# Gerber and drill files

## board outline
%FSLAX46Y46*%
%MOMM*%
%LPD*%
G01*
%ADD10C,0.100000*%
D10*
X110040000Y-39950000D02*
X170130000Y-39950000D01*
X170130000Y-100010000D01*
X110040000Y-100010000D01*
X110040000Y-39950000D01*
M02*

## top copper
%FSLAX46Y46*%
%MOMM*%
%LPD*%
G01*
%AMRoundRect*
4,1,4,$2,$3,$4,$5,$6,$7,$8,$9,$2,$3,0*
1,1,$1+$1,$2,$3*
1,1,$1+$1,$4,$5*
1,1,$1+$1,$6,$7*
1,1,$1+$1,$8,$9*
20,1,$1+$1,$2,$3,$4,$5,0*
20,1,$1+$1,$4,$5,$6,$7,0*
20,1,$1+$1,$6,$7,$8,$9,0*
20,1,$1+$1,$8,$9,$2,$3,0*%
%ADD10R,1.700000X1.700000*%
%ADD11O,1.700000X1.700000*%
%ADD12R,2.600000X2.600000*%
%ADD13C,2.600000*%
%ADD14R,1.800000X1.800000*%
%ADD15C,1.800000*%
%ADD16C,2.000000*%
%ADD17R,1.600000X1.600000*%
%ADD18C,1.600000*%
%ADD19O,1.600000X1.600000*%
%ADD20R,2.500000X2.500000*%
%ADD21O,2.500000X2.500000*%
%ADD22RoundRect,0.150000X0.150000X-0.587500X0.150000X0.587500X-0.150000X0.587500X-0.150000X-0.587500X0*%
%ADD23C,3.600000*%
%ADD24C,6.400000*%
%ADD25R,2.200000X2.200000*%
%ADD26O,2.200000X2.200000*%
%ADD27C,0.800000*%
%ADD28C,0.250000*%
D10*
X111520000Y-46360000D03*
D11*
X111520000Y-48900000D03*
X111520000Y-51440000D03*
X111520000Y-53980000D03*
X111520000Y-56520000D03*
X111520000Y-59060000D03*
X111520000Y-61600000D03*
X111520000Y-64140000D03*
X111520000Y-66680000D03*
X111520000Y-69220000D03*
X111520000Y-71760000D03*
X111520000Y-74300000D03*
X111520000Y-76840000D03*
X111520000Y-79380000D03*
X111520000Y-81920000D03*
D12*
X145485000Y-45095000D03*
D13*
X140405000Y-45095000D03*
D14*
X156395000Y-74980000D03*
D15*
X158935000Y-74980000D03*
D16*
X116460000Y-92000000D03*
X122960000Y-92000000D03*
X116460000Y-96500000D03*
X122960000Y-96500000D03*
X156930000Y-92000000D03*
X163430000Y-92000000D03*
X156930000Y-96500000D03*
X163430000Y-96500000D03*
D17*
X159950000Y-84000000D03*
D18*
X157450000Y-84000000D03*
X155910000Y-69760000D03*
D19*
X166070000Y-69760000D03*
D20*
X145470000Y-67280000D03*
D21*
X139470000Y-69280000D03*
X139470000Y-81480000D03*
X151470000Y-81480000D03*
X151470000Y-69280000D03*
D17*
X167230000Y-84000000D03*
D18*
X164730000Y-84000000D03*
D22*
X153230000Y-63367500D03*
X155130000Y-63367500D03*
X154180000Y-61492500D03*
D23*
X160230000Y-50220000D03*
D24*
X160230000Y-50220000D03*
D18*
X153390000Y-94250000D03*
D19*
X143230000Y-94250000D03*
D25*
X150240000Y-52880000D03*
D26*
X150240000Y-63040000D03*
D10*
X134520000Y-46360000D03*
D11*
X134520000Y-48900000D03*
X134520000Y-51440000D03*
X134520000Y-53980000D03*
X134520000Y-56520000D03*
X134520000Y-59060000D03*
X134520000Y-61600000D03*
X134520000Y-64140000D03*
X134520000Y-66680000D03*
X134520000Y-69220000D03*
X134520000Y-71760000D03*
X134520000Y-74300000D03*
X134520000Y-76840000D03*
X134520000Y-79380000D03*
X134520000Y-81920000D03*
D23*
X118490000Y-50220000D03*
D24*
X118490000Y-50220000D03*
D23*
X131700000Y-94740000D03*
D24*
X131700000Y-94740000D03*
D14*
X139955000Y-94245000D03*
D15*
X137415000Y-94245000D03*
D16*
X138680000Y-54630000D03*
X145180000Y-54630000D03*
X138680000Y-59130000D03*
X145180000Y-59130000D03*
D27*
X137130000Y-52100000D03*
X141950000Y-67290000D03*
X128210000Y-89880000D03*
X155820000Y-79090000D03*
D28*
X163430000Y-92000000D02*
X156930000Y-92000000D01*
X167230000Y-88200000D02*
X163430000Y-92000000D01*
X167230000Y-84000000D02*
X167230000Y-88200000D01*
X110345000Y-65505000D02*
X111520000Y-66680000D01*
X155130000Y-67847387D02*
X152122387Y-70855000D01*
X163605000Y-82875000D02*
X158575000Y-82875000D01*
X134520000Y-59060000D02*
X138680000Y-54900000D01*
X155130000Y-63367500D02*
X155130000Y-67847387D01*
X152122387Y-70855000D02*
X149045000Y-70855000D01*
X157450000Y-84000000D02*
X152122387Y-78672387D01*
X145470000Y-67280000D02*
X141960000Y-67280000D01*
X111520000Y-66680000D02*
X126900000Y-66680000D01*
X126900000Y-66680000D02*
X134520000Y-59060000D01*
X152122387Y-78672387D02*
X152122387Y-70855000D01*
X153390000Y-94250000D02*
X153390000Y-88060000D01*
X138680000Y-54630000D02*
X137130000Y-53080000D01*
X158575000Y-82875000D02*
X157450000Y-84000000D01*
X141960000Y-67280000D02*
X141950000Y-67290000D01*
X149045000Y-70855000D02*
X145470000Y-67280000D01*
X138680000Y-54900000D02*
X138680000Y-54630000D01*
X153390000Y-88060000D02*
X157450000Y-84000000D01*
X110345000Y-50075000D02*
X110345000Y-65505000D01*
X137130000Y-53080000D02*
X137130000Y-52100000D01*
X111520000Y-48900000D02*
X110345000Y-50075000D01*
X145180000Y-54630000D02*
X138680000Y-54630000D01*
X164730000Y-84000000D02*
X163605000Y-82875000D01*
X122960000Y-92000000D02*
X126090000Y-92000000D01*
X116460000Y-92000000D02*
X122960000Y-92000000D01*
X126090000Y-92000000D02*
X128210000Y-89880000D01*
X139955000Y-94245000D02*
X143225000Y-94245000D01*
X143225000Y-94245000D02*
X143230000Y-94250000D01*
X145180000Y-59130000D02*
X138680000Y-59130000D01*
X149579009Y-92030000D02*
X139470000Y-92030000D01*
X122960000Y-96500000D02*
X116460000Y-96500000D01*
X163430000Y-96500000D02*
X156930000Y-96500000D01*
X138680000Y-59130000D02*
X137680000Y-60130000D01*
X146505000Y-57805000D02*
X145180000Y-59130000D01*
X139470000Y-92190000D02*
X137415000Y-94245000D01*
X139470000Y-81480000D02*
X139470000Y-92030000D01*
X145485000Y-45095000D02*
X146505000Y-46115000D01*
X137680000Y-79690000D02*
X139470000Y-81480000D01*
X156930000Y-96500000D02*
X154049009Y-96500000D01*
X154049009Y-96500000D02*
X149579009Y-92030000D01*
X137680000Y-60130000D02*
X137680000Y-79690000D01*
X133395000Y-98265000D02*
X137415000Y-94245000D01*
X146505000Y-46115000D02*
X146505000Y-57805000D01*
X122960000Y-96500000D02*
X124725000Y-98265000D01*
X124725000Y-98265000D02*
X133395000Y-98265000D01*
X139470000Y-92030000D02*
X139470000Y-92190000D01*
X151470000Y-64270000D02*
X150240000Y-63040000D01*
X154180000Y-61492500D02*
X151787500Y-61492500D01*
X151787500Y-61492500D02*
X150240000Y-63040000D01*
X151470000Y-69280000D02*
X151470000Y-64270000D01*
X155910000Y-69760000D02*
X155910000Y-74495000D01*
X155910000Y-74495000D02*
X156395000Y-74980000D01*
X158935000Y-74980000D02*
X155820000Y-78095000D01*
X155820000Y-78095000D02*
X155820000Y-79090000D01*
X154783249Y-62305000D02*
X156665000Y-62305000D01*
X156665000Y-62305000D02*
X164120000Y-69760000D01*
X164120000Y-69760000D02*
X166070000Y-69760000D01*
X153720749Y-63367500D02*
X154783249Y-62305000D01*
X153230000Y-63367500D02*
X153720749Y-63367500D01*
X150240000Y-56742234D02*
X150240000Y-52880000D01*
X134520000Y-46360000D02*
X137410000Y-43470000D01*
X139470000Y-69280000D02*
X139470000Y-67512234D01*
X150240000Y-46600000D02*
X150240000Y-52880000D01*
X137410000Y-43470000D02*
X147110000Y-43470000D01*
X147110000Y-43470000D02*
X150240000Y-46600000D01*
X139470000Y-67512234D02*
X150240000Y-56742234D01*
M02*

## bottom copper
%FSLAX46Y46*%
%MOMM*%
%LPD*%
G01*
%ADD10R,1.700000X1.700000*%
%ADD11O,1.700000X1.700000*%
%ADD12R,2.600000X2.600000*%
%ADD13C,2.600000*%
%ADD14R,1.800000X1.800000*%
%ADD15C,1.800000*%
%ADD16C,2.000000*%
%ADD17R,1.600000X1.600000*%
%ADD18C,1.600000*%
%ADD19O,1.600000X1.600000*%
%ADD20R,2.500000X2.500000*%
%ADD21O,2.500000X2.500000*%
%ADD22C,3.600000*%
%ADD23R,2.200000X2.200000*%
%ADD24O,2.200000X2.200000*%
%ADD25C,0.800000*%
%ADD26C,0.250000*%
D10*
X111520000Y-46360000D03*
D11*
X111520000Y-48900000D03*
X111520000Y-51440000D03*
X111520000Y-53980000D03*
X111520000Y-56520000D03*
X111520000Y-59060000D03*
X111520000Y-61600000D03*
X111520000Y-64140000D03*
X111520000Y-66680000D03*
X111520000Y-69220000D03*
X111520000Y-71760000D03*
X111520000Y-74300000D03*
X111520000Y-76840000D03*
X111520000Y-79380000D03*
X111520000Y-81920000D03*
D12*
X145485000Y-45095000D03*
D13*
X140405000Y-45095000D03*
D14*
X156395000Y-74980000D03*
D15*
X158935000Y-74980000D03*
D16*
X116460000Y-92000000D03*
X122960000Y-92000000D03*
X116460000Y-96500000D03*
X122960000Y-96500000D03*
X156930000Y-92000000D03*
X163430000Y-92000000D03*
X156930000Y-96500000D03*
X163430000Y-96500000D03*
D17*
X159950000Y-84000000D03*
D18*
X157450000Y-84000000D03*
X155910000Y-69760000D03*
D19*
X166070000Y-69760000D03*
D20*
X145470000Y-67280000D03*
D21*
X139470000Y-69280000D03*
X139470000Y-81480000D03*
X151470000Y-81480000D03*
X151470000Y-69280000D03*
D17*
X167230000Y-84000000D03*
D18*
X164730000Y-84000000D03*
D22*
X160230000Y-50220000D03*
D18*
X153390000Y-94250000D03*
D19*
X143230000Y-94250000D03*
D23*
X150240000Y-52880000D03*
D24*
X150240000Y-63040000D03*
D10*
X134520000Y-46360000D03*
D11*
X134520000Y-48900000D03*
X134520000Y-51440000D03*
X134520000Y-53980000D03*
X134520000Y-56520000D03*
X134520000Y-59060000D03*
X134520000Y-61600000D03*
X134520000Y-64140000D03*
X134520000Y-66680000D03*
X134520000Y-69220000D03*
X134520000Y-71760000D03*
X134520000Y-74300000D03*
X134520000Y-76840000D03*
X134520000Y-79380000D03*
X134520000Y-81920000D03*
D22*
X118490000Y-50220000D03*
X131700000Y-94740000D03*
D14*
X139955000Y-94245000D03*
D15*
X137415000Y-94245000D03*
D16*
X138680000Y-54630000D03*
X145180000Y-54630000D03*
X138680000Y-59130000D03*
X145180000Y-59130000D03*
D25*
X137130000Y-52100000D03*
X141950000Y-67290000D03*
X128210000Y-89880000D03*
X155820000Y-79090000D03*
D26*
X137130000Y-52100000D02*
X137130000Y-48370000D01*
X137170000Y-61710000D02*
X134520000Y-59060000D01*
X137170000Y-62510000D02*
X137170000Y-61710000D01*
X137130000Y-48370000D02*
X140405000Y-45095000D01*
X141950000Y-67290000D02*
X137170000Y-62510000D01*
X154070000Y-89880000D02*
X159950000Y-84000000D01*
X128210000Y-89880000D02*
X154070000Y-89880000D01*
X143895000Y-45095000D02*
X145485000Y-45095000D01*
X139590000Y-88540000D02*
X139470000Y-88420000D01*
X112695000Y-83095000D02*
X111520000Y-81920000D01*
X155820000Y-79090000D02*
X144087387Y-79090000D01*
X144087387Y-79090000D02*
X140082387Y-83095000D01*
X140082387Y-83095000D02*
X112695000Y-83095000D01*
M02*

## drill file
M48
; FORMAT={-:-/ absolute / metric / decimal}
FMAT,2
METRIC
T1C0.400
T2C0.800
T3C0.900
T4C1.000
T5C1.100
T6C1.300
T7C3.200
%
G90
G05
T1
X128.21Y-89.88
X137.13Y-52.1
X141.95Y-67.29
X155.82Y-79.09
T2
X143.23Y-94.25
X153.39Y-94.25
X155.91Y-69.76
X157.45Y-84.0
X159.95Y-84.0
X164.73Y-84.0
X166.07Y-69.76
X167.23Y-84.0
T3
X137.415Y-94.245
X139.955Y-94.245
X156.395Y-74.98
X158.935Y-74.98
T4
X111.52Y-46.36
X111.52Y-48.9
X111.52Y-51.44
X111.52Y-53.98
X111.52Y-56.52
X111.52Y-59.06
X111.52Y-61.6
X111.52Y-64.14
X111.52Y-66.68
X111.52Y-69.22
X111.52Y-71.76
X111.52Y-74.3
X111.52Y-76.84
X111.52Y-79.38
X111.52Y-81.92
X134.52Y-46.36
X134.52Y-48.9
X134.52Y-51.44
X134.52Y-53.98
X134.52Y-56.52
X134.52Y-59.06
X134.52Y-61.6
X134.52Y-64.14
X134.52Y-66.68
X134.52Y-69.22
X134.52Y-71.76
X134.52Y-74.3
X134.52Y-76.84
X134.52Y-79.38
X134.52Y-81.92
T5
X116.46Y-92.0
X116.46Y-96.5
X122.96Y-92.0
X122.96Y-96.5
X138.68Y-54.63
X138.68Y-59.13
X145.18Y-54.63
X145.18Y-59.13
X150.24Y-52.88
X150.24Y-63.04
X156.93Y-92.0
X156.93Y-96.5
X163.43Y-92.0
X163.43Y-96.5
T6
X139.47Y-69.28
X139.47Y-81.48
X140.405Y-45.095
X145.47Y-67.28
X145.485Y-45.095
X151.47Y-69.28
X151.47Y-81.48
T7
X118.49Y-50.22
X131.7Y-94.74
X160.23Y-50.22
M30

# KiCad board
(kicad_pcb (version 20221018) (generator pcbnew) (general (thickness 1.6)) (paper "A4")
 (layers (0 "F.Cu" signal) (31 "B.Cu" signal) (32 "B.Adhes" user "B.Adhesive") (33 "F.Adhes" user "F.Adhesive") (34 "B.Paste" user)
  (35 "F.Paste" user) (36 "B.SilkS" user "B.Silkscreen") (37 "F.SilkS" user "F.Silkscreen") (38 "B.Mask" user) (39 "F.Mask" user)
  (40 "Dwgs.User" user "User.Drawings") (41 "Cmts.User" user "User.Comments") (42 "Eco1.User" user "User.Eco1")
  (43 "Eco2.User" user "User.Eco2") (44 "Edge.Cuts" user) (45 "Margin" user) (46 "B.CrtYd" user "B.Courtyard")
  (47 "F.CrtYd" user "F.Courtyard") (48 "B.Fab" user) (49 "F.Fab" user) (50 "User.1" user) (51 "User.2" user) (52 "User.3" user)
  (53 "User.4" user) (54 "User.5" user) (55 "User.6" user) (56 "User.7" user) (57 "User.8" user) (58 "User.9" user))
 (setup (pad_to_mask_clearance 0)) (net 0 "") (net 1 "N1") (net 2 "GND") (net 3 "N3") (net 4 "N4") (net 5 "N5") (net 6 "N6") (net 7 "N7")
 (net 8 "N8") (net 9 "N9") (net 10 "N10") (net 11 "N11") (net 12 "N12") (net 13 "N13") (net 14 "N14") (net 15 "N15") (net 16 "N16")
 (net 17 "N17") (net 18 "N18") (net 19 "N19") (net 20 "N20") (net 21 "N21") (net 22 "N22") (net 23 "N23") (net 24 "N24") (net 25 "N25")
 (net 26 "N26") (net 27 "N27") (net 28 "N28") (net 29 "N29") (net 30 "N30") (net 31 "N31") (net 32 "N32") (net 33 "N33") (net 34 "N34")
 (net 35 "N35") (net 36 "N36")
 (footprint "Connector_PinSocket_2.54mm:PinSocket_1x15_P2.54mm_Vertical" (layer "F.Cu") (at 111.52 46.36)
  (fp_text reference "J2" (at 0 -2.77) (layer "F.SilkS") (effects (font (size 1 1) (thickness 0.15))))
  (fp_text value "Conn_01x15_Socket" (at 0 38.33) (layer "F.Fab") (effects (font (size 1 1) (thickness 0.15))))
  (pad "1" thru_hole rect (at 0 0) (size 1.7 1.7) (drill 1) (layers "*.Cu" "*.Mask") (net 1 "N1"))
  (pad "2" thru_hole oval (at 0 2.54) (size 1.7 1.7) (drill 1) (layers "*.Cu" "*.Mask") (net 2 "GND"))
  (pad "3" thru_hole oval (at 0 5.08) (size 1.7 1.7) (drill 1) (layers "*.Cu" "*.Mask") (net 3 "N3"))
  (pad "4" thru_hole oval (at 0 7.62) (size 1.7 1.7) (drill 1) (layers "*.Cu" "*.Mask") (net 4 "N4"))
  (pad "5" thru_hole oval (at 0 10.16) (size 1.7 1.7) (drill 1) (layers "*.Cu" "*.Mask") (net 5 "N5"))
  (pad "6" thru_hole oval (at 0 12.7) (size 1.7 1.7) (drill 1) (layers "*.Cu" "*.Mask") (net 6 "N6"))
  (pad "7" thru_hole oval (at 0 15.24) (size 1.7 1.7) (drill 1) (layers "*.Cu" "*.Mask") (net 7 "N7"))
  (pad "8" thru_hole oval (at 0 17.78) (size 1.7 1.7) (drill 1) (layers "*.Cu" "*.Mask") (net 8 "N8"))
  (pad "9" thru_hole oval (at 0 20.32) (size 1.7 1.7) (drill 1) (layers "*.Cu" "*.Mask") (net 2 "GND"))
  (pad "10" thru_hole oval (at 0 22.86) (size 1.7 1.7) (drill 1) (layers "*.Cu" "*.Mask") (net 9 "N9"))
  (pad "11" thru_hole oval (at 0 25.4) (size 1.7 1.7) (drill 1) (layers "*.Cu" "*.Mask") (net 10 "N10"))
  (pad "12" thru_hole oval (at 0 27.94) (size 1.7 1.7) (drill 1) (layers "*.Cu" "*.Mask") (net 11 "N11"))
  (pad "13" thru_hole oval (at 0 30.48) (size 1.7 1.7) (drill 1) (layers "*.Cu" "*.Mask") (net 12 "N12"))
  (pad "14" thru_hole oval (at 0 33.02) (size 1.7 1.7) (drill 1) (layers "*.Cu" "*.Mask") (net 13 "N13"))
  (pad "15" thru_hole oval (at 0 35.56) (size 1.7 1.7) (drill 1) (layers "*.Cu" "*.Mask") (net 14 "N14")))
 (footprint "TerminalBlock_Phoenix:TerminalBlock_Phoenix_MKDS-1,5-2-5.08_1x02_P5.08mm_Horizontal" (layer "F.Cu") (at 145.485 45.095 180)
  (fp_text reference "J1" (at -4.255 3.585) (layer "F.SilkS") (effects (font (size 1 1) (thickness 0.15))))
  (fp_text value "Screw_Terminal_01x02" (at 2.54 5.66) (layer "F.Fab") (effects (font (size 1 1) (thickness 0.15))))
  (pad "1" thru_hole rect (at 0 0 180) (size 2.6 2.6) (drill 1.3) (layers "*.Cu" "*.Mask") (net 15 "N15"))
  (pad "2" thru_hole circle (at 5.08 0 180) (size 2.6 2.6) (drill 1.3) (layers "*.Cu" "*.Mask") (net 2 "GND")))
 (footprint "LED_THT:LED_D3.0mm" (layer "F.Cu") (at 156.395 74.98)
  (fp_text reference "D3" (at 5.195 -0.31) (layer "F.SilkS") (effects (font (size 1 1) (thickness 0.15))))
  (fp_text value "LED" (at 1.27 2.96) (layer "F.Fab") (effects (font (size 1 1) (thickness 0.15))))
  (pad "1" thru_hole rect (at 0 0) (size 1.8 1.8) (drill 0.9) (layers "*.Cu" "*.Mask") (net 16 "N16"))
  (pad "2" thru_hole circle (at 2.54 0) (size 1.8 1.8) (drill 0.9) (layers "*.Cu" "*.Mask") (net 14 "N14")))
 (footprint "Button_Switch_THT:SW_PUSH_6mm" (layer "F.Cu") (at 116.46 92)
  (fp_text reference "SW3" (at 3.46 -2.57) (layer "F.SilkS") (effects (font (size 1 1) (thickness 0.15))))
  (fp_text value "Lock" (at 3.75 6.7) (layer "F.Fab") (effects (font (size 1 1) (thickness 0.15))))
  (pad "1" thru_hole circle (at 0 0 90) (size 2 2) (drill 1.1) (layers "*.Cu" "*.Mask") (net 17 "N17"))
  (pad "1" thru_hole circle (at 6.5 0 90) (size 2 2) (drill 1.1) (layers "*.Cu" "*.Mask") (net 17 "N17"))
  (pad "2" thru_hole circle (at 0 4.5 90) (size 2 2) (drill 1.1) (layers "*.Cu" "*.Mask") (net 15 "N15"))
  (pad "2" thru_hole circle (at 6.5 4.5 90) (size 2 2) (drill 1.1) (layers "*.Cu" "*.Mask") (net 15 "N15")))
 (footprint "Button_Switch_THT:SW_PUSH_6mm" (layer "F.Cu") (at 156.93 92)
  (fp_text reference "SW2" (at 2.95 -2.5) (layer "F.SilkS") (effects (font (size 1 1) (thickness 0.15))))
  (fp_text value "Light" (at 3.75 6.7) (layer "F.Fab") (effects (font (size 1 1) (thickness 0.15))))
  (pad "1" thru_hole circle (at 0 0 90) (size 2 2) (drill 1.1) (layers "*.Cu" "*.Mask") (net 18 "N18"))
  (pad "1" thru_hole circle (at 6.5 0 90) (size 2 2) (drill 1.1) (layers "*.Cu" "*.Mask") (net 18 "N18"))
  (pad "2" thru_hole circle (at 0 4.5 90) (size 2 2) (drill 1.1) (layers "*.Cu" "*.Mask") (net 15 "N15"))
  (pad "2" thru_hole circle (at 6.5 4.5 90) (size 2 2) (drill 1.1) (layers "*.Cu" "*.Mask") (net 15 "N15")))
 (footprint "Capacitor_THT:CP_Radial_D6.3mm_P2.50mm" (layer "F.Cu") (at 159.95 84 180)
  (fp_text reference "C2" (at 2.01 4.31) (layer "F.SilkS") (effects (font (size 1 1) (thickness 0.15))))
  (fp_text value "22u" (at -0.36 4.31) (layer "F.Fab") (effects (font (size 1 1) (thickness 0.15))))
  (pad "1" thru_hole rect (at 0 0 180) (size 1.6 1.6) (drill 0.8) (layers "*.Cu" "*.Mask") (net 17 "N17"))
  (pad "2" thru_hole circle (at 2.5 0 180) (size 1.6 1.6) (drill 0.8) (layers "*.Cu" "*.Mask") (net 2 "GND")))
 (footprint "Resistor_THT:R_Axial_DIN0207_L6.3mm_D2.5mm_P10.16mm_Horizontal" (layer "F.Cu") (at 155.91 69.76)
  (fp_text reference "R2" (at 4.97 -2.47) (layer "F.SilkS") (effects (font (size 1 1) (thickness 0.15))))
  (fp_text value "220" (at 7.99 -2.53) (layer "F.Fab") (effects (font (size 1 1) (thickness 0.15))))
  (pad "1" thru_hole circle (at 0 0) (size 1.6 1.6) (drill 0.8) (layers "*.Cu" "*.Mask") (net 16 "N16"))
  (pad "2" thru_hole oval (at 10.16 0) (size 1.6 1.6) (drill 0.8) (layers "*.Cu" "*.Mask") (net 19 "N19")))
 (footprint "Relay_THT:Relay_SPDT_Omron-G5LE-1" (layer "F.Cu") (at 145.47 67.28)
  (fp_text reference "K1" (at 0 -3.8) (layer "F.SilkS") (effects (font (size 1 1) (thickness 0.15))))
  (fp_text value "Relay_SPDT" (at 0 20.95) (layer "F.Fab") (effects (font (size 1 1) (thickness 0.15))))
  (pad "1" thru_hole rect (at 0 0) (size 2.5 2.5) (drill 1.3) (layers "*.Cu" "*.Mask") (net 2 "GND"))
  (pad "2" thru_hole oval (at -6 2) (size 2.5 2.5) (drill 1.3) (layers "*.Cu" "*.Mask") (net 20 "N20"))
  (pad "3" thru_hole oval (at -6 14.2) (size 2.5 2.5) (drill 1.3) (layers "*.Cu" "*.Mask") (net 15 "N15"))
  (pad "4" thru_hole oval (at 6 14.2) (size 2.5 2.5) (drill 1.3) (layers "*.Cu" "*.Mask") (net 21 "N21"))
  (pad "5" thru_hole oval (at 6 2) (size 2.5 2.5) (drill 1.3) (layers "*.Cu" "*.Mask") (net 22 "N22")))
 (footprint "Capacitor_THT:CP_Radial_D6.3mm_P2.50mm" (layer "F.Cu") (at 167.23 84 180)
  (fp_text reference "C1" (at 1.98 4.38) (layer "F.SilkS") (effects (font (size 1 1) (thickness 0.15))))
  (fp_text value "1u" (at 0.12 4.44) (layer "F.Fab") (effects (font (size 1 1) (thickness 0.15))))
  (pad "1" thru_hole rect (at 0 0 180) (size 1.6 1.6) (drill 0.8) (layers "*.Cu" "*.Mask") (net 18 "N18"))
  (pad "2" thru_hole circle (at 2.5 0 180) (size 1.6 1.6) (drill 0.8) (layers "*.Cu" "*.Mask") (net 2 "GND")))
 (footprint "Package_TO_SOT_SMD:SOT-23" (layer "F.Cu") (at 154.18 62.43 90)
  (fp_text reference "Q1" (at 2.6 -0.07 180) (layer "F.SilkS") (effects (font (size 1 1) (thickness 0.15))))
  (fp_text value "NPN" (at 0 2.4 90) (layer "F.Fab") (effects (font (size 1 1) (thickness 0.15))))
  (pad "1" smd roundrect (at -0.9375 -0.95 90) (size 1.475 0.6) (layers "F.Cu" "F.Paste" "F.Mask") (roundrect_rratio 0.25) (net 19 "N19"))
  (pad "2" smd roundrect (at -0.9375 0.95 90) (size 1.475 0.6) (layers "F.Cu" "F.Paste" "F.Mask") (roundrect_rratio 0.25) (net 2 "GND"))
  (pad "3" smd roundrect (at 0.9375 0 90) (size 1.475 0.6) (layers "F.Cu" "F.Paste" "F.Mask") (roundrect_rratio 0.25) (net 22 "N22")))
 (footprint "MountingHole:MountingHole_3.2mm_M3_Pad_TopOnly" (layer "F.Cu") (at 160.23 50.22)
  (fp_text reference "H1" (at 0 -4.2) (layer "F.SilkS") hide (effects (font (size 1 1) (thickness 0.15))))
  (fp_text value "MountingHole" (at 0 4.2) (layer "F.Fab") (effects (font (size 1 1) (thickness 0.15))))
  (pad "1" thru_hole circle (at 0 0) (size 3.6 3.6) (drill 3.2) (layers "*.Cu" "*.Mask"))
  (pad "1" connect circle (at 0 0) (size 6.4 6.4) (layers "F.Cu" "F.Mask")))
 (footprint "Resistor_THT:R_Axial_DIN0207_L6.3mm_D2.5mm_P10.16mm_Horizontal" (layer "F.Cu") (at 153.39 94.25 180)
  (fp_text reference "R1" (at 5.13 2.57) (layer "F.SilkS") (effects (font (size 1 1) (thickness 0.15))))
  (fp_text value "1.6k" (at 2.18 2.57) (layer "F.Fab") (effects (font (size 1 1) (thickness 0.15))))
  (pad "1" thru_hole circle (at 0 0 180) (size 1.6 1.6) (drill 0.8) (layers "*.Cu" "*.Mask") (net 2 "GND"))
  (pad "2" thru_hole oval (at 10.16 0 180) (size 1.6 1.6) (drill 0.8) (layers "*.Cu" "*.Mask") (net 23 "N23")))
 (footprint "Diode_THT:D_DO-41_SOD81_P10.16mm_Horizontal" (layer "F.Cu") (at 150.24 52.88 -90)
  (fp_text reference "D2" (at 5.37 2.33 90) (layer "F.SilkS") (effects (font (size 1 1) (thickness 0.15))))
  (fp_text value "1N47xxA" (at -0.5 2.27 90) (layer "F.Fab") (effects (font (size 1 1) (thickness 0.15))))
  (pad "1" thru_hole rect (at 0 0 270) (size 2.2 2.2) (drill 1.1) (layers "*.Cu" "*.Mask") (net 20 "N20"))
  (pad "2" thru_hole oval (at 10.16 0 270) (size 2.2 2.2) (drill 1.1) (layers "*.Cu" "*.Mask") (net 22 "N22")))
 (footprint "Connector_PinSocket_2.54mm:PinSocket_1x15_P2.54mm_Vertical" (layer "F.Cu") (at 134.52 46.36)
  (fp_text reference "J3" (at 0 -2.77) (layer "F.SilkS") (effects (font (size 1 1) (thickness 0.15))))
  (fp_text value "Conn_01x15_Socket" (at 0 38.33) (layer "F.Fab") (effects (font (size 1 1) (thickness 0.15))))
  (pad "1" thru_hole rect (at 0 0) (size 1.7 1.7) (drill 1) (layers "*.Cu" "*.Mask") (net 20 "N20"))
  (pad "2" thru_hole oval (at 0 2.54) (size 1.7 1.7) (drill 1) (layers "*.Cu" "*.Mask") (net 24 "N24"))
  (pad "3" thru_hole oval (at 0 5.08) (size 1.7 1.7) (drill 1) (layers "*.Cu" "*.Mask") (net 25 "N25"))
  (pad "4" thru_hole oval (at 0 7.62) (size 1.7 1.7) (drill 1) (layers "*.Cu" "*.Mask") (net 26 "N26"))
  (pad "5" thru_hole oval (at 0 10.16) (size 1.7 1.7) (drill 1) (layers "*.Cu" "*.Mask") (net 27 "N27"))
  (pad "6" thru_hole oval (at 0 12.7) (size 1.7 1.7) (drill 1) (layers "*.Cu" "*.Mask") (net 2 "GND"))
  (pad "7" thru_hole oval (at 0 15.24) (size 1.7 1.7) (drill 1) (layers "*.Cu" "*.Mask") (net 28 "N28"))
  (pad "8" thru_hole oval (at 0 17.78) (size 1.7 1.7) (drill 1) (layers "*.Cu" "*.Mask") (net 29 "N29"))
  (pad "9" thru_hole oval (at 0 20.32) (size 1.7 1.7) (drill 1) (layers "*.Cu" "*.Mask") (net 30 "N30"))
  (pad "10" thru_hole oval (at 0 22.86) (size 1.7 1.7) (drill 1) (layers "*.Cu" "*.Mask") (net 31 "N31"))
  (pad "11" thru_hole oval (at 0 25.4) (size 1.7 1.7) (drill 1) (layers "*.Cu" "*.Mask") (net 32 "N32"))
  (pad "12" thru_hole oval (at 0 27.94) (size 1.7 1.7) (drill 1) (layers "*.Cu" "*.Mask") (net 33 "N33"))
  (pad "13" thru_hole oval (at 0 30.48) (size 1.7 1.7) (drill 1) (layers "*.Cu" "*.Mask") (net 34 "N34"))
  (pad "14" thru_hole oval (at 0 33.02) (size 1.7 1.7) (drill 1) (layers "*.Cu" "*.Mask") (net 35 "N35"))
  (pad "15" thru_hole oval (at 0 35.56) (size 1.7 1.7) (drill 1) (layers "*.Cu" "*.Mask") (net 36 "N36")))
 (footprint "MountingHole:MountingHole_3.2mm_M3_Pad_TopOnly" (layer "F.Cu") (at 118.49 50.22)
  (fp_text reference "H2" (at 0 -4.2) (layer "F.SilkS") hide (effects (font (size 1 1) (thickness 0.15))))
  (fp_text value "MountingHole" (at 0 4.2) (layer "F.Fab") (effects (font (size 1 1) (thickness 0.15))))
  (pad "1" thru_hole circle (at 0 0) (size 3.6 3.6) (drill 3.2) (layers "*.Cu" "*.Mask"))
  (pad "1" connect circle (at 0 0) (size 6.4 6.4) (layers "F.Cu" "F.Mask")))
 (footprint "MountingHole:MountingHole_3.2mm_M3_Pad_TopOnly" (layer "F.Cu") (at 131.7 94.74)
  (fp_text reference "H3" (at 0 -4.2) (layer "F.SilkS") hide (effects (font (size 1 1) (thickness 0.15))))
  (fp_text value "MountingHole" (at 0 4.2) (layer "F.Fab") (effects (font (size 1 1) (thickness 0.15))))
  (pad "1" thru_hole circle (at 0 0) (size 3.6 3.6) (drill 3.2) (layers "*.Cu" "*.Mask"))
  (pad "1" connect circle (at 0 0) (size 6.4 6.4) (layers "F.Cu" "F.Mask")))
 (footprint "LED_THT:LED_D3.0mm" (layer "F.Cu") (at 139.955 94.245 180)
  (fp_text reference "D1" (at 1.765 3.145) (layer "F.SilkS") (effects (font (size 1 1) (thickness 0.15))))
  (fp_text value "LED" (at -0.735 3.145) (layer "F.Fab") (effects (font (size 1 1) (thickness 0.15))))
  (pad "1" thru_hole rect (at 0 0 180) (size 1.8 1.8) (drill 0.9) (layers "*.Cu" "*.Mask") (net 23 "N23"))
  (pad "2" thru_hole circle (at 2.54 0 180) (size 1.8 1.8) (drill 0.9) (layers "*.Cu" "*.Mask") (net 15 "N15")))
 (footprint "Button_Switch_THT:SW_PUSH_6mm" (layer "F.Cu") (at 138.68 54.63)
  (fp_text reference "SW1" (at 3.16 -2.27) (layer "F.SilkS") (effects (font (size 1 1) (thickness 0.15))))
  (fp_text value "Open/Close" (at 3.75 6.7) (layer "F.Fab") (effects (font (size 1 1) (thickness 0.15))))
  (pad "1" thru_hole circle (at 0 0 90) (size 2 2) (drill 1.1) (layers "*.Cu" "*.Mask") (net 2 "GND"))
  (pad "1" thru_hole circle (at 6.5 0 90) (size 2 2) (drill 1.1) (layers "*.Cu" "*.Mask") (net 2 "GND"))
  (pad "2" thru_hole circle (at 0 4.5 90) (size 2 2) (drill 1.1) (layers "*.Cu" "*.Mask") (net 15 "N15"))
  (pad "2" thru_hole circle (at 6.5 4.5 90) (size 2 2) (drill 1.1) (layers "*.Cu" "*.Mask") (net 15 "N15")))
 (gr_rect (start 110.04 39.95) (end 170.13 100.01) (stroke (width 0.1) (type default)) (fill none) (layer "Edge.Cuts"))
 (segment (start 163.43 92) (end 156.93 92) (width 0.25) (layer "F.Cu") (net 18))
 (segment (start 167.23 88.2) (end 163.43 92) (width 0.25) (layer "F.Cu") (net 18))
 (segment (start 167.23 84) (end 167.23 88.2) (width 0.25) (layer "F.Cu") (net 18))
 (segment (start 110.345 65.505) (end 111.52 66.68) (width 0.25) (layer "F.Cu") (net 2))
 (segment (start 155.13 67.847387) (end 152.122387 70.855) (width 0.25) (layer "F.Cu") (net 2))
 (segment (start 163.605 82.875) (end 158.575 82.875) (width 0.25) (layer "F.Cu") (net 2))
 (segment (start 134.52 59.06) (end 138.68 54.9) (width 0.25) (layer "F.Cu") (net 2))
 (segment (start 155.13 63.3675) (end 155.13 67.847387) (width 0.25) (layer "F.Cu") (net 2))
 (segment (start 152.122387 70.855) (end 149.045 70.855) (width 0.25) (layer "F.Cu") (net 2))
 (segment (start 157.45 84) (end 152.122387 78.672387) (width 0.25) (layer "F.Cu") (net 2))
 (segment (start 145.47 67.28) (end 141.96 67.28) (width 0.25) (layer "F.Cu") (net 2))
 (segment (start 111.52 66.68) (end 126.9 66.68) (width 0.25) (layer "F.Cu") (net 2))
 (segment (start 126.9 66.68) (end 134.52 59.06) (width 0.25) (layer "F.Cu") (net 2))
 (segment (start 152.122387 78.672387) (end 152.122387 70.855) (width 0.25) (layer "F.Cu") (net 2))
 (segment (start 153.39 94.25) (end 153.39 88.06) (width 0.25) (layer "F.Cu") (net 2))
 (segment (start 138.68 54.63) (end 137.13 53.08) (width 0.25) (layer "F.Cu") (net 2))
 (segment (start 158.575 82.875) (end 157.45 84) (width 0.25) (layer "F.Cu") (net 2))
 (segment (start 141.96 67.28) (end 141.95 67.29) (width 0.25) (layer "F.Cu") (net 2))
 (segment (start 149.045 70.855) (end 145.47 67.28) (width 0.25) (layer "F.Cu") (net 2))
 (segment (start 138.68 54.9) (end 138.68 54.63) (width 0.25) (layer "F.Cu") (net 2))
 (segment (start 153.39 88.06) (end 157.45 84) (width 0.25) (layer "F.Cu") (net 2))
 (segment (start 110.345 50.075) (end 110.345 65.505) (width 0.25) (layer "F.Cu") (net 2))
 (segment (start 137.13 53.08) (end 137.13 52.1) (width 0.25) (layer "F.Cu") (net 2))
 (segment (start 111.52 48.9) (end 110.345 50.075) (width 0.25) (layer "F.Cu") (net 2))
 (segment (start 145.18 54.63) (end 138.68 54.63) (width 0.25) (layer "F.Cu") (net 2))
 (segment (start 164.73 84) (end 163.605 82.875) (width 0.25) (layer "F.Cu") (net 2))
 (via (at 137.13 52.1) (size 0.8) (drill 0.4) (layers "F.Cu" "B.Cu") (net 2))
 (via (at 141.95 67.29) (size 0.8) (drill 0.4) (layers "F.Cu" "B.Cu") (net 2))
 (segment (start 137.13 52.1) (end 137.13 48.37) (width 0.25) (layer "B.Cu") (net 2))
 (segment (start 137.17 61.71) (end 134.52 59.06) (width 0.25) (layer "B.Cu") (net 2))
 (segment (start 137.17 62.51) (end 137.17 61.71) (width 0.25) (layer "B.Cu") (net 2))
 (segment (start 137.13 48.37) (end 140.405 45.095) (width 0.25) (layer "B.Cu") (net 2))
 (segment (start 141.95 67.29) (end 137.17 62.51) (width 0.25) (layer "B.Cu") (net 2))
 (segment (start 122.96 92) (end 126.09 92) (width 0.25) (layer "F.Cu") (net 17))
 (segment (start 116.46 92) (end 122.96 92) (width 0.25) (layer "F.Cu") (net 17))
 (segment (start 126.09 92) (end 128.21 89.88) (width 0.25) (layer "F.Cu") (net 17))
 (via (at 128.21 89.88) (size 0.8) (drill 0.4) (layers "F.Cu" "B.Cu") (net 17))
 (segment (start 154.07 89.88) (end 159.95 84) (width 0.25) (layer "B.Cu") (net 17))
 (segment (start 128.21 89.88) (end 154.07 89.88) (width 0.25) (layer "B.Cu") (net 17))
 (segment (start 139.955 94.245) (end 143.225 94.245) (width 0.25) (layer "F.Cu") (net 23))
 (segment (start 143.225 94.245) (end 143.23 94.25) (width 0.25) (layer "F.Cu") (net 23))
 (segment (start 145.18 59.13) (end 138.68 59.13) (width 0.25) (layer "F.Cu") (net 15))
 (segment (start 149.579009 92.03) (end 139.47 92.03) (width 0.25) (layer "F.Cu") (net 15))
 (segment (start 122.96 96.5) (end 116.46 96.5) (width 0.25) (layer "F.Cu") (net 15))
 (segment (start 163.43 96.5) (end 156.93 96.5) (width 0.25) (layer "F.Cu") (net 15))
 (segment (start 138.68 59.13) (end 137.68 60.13) (width 0.25) (layer "F.Cu") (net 15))
 (segment (start 146.505 57.805) (end 145.18 59.13) (width 0.25) (layer "F.Cu") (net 15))
 (segment (start 139.47 92.19) (end 137.415 94.245) (width 0.25) (layer "F.Cu") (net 15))
 (segment (start 139.47 81.48) (end 139.47 92.03) (width 0.25) (layer "F.Cu") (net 15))
 (segment (start 145.485 45.095) (end 146.505 46.115) (width 0.25) (layer "F.Cu") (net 15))
 (segment (start 137.68 79.69) (end 139.47 81.48) (width 0.25) (layer "F.Cu") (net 15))
 (segment (start 156.93 96.5) (end 154.049009 96.5) (width 0.25) (layer "F.Cu") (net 15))
 (segment (start 154.049009 96.5) (end 149.579009 92.03) (width 0.25) (layer "F.Cu") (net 15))
 (segment (start 137.68 60.13) (end 137.68 79.69) (width 0.25) (layer "F.Cu") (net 15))
 (segment (start 133.395 98.265) (end 137.415 94.245) (width 0.25) (layer "F.Cu") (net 15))
 (segment (start 146.505 46.115) (end 146.505 57.805) (width 0.25) (layer "F.Cu") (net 15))
 (segment (start 122.96 96.5) (end 124.725 98.265) (width 0.25) (layer "F.Cu") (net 15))
 (segment (start 124.725 98.265) (end 133.395 98.265) (width 0.25) (layer "F.Cu") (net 15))
 (segment (start 139.47 92.03) (end 139.47 92.19) (width 0.25) (layer "F.Cu") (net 15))
 (segment (start 143.895 45.095) (end 145.485 45.095) (width 0.25) (layer "B.Cu") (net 15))
 (segment (start 139.59 88.54) (end 139.47 88.42) (width 0.25) (layer "B.Cu") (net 15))
 (segment (start 151.47 64.27) (end 150.24 63.04) (width 0.25) (layer "F.Cu") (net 22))
 (segment (start 154.18 61.4925) (end 151.7875 61.4925) (width 0.25) (layer "F.Cu") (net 22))
 (segment (start 151.7875 61.4925) (end 150.24 63.04) (width 0.25) (layer "F.Cu") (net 22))
 (segment (start 151.47 69.28) (end 151.47 64.27) (width 0.25) (layer "F.Cu") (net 22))
 (segment (start 155.91 69.76) (end 155.91 74.495) (width 0.25) (layer "F.Cu") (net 16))
 (segment (start 155.91 74.495) (end 156.395 74.98) (width 0.25) (layer "F.Cu") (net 16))
 (segment (start 158.935 74.98) (end 155.82 78.095) (width 0.25) (layer "F.Cu") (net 14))
 (segment (start 155.82 78.095) (end 155.82 79.09) (width 0.25) (layer "F.Cu") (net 14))
 (via (at 155.82 79.09) (size 0.8) (drill 0.4) (layers "F.Cu" "B.Cu") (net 14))
 (segment (start 112.695 83.095) (end 111.52 81.92) (width 0.25) (layer "B.Cu") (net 14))
 (segment (start 155.82 79.09) (end 144.087387 79.09) (width 0.25) (layer "B.Cu") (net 14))
 (segment (start 144.087387 79.09) (end 140.082387 83.095) (width 0.25) (layer "B.Cu") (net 14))
 (segment (start 140.082387 83.095) (end 112.695 83.095) (width 0.25) (layer "B.Cu") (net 14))
 (segment (start 154.783249 62.305) (end 156.665 62.305) (width 0.25) (layer "F.Cu") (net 19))
 (segment (start 156.665 62.305) (end 164.12 69.76) (width 0.25) (layer "F.Cu") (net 19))
 (segment (start 164.12 69.76) (end 166.07 69.76) (width 0.25) (layer "F.Cu") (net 19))
 (segment (start 153.720749 63.3675) (end 154.783249 62.305) (width 0.25) (layer "F.Cu") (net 19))
 (segment (start 153.23 63.3675) (end 153.720749 63.3675) (width 0.25) (layer "F.Cu") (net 19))
 (segment (start 150.24 56.742234) (end 150.24 52.88) (width 0.25) (layer "F.Cu") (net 20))
 (segment (start 134.52 46.36) (end 137.41 43.47) (width 0.25) (layer "F.Cu") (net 20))
 (segment (start 139.47 69.28) (end 139.47 67.512234) (width 0.25) (layer "F.Cu") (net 20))
 (segment (start 150.24 46.6) (end 150.24 52.88) (width 0.25) (layer "F.Cu") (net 20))
 (segment (start 137.41 43.47) (end 147.11 43.47) (width 0.25) (layer "F.Cu") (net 20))
 (segment (start 147.11 43.47) (end 150.24 46.6) (width 0.25) (layer "F.Cu") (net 20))
 (segment (start 139.47 67.512234) (end 150.24 56.742234) (width 0.25) (layer "F.Cu") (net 20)))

